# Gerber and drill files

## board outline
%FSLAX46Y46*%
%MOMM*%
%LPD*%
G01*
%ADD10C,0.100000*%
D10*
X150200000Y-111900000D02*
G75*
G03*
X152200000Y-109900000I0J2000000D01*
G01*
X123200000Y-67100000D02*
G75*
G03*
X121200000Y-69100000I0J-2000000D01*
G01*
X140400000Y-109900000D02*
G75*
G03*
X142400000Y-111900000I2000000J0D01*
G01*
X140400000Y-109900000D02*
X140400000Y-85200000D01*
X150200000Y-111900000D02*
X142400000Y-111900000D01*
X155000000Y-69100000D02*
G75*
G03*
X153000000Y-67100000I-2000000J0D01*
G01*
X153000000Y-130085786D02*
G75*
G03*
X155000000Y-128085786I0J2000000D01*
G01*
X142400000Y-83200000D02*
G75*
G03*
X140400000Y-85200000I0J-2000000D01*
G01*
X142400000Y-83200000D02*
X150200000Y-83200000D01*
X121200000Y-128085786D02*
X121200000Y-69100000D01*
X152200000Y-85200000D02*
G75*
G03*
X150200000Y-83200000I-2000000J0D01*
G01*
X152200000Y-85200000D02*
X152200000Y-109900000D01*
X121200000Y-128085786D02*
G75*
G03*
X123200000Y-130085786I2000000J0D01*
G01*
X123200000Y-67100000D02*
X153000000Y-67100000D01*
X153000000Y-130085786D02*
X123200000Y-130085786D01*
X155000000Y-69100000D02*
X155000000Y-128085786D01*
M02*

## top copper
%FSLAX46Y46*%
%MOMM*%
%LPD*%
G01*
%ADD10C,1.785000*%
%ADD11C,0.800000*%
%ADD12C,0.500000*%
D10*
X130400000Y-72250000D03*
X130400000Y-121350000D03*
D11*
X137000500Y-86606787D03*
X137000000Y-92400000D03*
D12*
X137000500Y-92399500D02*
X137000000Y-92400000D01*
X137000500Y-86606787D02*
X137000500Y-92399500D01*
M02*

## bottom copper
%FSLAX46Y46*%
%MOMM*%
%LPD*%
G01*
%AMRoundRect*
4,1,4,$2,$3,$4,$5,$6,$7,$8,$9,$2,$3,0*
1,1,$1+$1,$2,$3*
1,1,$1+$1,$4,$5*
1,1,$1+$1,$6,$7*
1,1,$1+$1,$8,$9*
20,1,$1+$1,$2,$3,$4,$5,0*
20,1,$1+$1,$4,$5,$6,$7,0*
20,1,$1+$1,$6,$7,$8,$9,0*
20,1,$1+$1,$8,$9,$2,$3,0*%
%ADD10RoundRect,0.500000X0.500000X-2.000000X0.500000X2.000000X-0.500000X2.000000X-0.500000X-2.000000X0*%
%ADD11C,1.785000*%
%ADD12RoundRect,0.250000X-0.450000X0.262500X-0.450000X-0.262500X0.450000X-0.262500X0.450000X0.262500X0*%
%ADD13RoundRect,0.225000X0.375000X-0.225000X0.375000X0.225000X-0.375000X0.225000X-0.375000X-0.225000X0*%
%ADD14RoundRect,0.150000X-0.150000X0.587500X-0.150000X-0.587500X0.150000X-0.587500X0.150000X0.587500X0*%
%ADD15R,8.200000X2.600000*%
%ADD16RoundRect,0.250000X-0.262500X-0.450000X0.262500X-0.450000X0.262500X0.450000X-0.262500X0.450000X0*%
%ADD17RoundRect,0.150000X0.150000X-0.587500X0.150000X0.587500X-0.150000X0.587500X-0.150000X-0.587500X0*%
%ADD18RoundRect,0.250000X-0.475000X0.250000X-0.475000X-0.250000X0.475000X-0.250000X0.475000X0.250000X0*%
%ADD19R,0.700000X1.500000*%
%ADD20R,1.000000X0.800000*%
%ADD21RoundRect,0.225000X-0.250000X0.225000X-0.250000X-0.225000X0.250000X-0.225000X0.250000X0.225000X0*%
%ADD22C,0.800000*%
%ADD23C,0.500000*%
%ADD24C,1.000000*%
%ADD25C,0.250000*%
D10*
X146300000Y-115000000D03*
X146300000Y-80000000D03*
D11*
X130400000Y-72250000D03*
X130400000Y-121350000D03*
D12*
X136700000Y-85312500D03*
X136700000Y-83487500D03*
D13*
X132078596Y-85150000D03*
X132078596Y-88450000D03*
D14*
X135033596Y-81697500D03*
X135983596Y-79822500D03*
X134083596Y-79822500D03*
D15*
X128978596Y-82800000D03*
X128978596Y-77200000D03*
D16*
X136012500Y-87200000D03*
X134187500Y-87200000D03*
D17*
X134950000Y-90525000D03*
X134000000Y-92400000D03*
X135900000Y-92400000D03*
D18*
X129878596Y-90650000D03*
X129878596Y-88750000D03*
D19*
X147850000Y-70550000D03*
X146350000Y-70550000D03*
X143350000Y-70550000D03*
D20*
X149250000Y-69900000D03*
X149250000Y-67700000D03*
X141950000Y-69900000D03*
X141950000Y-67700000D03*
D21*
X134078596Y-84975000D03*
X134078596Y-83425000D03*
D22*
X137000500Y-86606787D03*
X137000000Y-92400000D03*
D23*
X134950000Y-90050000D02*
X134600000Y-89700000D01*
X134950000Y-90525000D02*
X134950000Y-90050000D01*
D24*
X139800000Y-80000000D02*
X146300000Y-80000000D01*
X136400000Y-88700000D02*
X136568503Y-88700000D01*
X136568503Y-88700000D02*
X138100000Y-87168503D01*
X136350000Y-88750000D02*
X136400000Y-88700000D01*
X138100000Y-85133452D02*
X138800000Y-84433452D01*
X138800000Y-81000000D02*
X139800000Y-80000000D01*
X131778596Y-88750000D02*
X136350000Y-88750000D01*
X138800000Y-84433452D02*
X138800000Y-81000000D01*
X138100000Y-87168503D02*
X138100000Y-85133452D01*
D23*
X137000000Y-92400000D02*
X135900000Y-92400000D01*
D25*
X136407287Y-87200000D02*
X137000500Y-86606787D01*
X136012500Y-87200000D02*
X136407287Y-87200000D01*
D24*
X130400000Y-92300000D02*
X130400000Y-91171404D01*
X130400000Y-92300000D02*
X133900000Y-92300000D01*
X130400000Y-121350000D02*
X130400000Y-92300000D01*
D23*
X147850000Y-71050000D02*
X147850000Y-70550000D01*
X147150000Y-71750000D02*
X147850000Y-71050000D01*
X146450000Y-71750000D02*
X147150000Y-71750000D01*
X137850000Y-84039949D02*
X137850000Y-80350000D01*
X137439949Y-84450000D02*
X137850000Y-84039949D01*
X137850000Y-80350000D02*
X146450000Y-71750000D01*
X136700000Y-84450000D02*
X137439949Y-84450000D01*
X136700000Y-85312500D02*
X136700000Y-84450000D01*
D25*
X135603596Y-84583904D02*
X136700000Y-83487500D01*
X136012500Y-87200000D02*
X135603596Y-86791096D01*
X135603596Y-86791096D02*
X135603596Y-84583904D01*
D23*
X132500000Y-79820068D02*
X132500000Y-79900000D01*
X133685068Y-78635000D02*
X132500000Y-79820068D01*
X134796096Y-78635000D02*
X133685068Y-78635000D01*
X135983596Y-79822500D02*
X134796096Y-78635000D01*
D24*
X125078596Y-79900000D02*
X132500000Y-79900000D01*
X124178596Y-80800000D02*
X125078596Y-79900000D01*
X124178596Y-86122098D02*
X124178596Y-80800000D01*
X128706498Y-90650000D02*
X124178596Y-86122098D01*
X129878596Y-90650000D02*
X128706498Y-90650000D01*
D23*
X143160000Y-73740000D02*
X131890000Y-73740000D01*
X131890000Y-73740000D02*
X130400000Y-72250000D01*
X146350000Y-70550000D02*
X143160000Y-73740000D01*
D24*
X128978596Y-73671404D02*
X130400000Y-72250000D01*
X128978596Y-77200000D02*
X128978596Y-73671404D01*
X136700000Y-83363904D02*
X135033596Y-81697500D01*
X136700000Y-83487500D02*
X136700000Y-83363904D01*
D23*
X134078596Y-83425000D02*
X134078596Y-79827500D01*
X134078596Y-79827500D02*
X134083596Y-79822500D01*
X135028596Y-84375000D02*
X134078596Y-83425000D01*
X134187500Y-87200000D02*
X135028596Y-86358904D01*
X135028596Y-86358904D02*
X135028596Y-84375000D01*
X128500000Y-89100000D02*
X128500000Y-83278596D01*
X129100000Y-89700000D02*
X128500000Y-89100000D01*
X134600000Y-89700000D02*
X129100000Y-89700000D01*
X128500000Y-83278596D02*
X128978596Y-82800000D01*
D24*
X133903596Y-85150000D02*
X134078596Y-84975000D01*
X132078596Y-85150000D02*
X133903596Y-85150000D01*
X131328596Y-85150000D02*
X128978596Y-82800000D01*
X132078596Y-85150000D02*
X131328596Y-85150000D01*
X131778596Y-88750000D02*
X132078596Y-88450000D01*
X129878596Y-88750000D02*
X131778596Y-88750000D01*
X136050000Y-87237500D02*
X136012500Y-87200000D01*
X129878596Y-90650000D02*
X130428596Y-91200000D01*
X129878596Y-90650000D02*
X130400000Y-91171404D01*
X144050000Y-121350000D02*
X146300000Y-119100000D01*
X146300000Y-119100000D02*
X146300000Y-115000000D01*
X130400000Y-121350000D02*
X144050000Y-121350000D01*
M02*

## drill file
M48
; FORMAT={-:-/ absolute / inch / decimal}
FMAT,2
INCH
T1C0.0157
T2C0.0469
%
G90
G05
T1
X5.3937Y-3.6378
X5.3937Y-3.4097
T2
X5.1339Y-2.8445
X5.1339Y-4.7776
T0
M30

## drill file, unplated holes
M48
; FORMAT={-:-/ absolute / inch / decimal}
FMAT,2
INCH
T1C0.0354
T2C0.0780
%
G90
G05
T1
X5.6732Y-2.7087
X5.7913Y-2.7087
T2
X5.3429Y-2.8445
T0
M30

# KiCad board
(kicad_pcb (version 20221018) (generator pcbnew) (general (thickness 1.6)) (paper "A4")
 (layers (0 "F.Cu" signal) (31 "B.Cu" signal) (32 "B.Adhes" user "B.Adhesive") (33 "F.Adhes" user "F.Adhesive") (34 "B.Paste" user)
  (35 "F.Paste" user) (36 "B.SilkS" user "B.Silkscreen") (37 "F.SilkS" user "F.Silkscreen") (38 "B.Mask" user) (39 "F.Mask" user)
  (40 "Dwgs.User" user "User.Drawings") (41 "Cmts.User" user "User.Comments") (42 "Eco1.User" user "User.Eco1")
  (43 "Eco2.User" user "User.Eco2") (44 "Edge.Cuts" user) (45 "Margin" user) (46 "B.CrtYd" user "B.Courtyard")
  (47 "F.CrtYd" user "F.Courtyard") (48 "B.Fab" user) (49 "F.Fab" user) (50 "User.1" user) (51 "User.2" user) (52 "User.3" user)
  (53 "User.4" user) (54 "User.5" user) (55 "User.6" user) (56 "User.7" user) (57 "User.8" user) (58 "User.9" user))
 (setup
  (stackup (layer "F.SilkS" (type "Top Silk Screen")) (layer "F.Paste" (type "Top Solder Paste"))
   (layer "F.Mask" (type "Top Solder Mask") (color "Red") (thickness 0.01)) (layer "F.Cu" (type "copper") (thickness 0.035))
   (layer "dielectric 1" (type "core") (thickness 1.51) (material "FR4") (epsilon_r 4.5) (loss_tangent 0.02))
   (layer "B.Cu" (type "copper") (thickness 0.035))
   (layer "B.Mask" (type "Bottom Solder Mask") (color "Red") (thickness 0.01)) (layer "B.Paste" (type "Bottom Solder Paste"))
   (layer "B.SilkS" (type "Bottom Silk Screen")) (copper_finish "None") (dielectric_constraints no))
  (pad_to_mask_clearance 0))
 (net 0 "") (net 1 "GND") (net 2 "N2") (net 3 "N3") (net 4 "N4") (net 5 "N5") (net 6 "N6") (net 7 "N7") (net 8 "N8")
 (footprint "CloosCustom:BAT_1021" (layer "F.Cu") (at 130.4 96.8 -90)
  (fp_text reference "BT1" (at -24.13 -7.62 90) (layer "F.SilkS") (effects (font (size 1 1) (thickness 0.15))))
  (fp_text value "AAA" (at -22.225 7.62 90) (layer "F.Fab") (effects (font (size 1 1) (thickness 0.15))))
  (pad "" np_thru_hole circle (at -24.55 -5.31 270) (size 1.98 1.98) (drill 1.98) (layers "*.Cu" "*.Mask"))
  (pad "N" thru_hole circle (at 24.55 0 270) (size 1.785 1.785) (drill 1.19) (layers "*.Cu" "*.Mask") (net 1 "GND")
   (solder_mask_margin 0.102))
  (pad "P" thru_hole circle (at -24.55 0 270) (size 1.785 1.785) (drill 1.19) (layers "*.Cu" "*.Mask") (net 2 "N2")
   (solder_mask_margin 0.102)))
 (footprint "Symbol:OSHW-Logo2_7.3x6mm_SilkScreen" (layer "F.Cu") (at 150.6 78.7)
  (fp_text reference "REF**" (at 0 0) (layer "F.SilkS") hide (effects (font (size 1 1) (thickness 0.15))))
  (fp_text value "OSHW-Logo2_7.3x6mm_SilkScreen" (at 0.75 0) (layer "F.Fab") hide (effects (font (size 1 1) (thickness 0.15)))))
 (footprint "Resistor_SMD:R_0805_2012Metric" (layer "B.Cu") (at 136.7 84.4 -90)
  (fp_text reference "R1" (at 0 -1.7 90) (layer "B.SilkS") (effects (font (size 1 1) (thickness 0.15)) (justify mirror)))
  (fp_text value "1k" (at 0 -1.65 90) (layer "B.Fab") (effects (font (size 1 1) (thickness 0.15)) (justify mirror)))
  (pad "1" smd roundrect (at -0.9125 0 270) (size 1.025 1.4) (layers "B.Cu" "B.Paste" "B.Mask") (roundrect_rratio 0.243902439) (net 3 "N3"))
  (pad "2" smd roundrect (at 0.9125 0 270) (size 1.025 1.4) (layers "B.Cu" "B.Paste" "B.Mask") (roundrect_rratio 0.243902439) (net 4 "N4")))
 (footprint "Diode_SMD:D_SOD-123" (layer "B.Cu") (at 132.078596 86.8 90)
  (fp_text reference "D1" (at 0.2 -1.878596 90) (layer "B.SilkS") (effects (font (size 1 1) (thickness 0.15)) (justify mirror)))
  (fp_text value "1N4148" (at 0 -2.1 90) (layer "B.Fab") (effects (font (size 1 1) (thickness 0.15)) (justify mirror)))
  (pad "1" smd roundrect (at -1.65 0 90) (size 0.9 1.2) (layers "B.Cu" "B.Paste" "B.Mask") (roundrect_rratio 0.25) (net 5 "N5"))
  (pad "2" smd roundrect (at 1.65 0 90) (size 0.9 1.2) (layers "B.Cu" "B.Paste" "B.Mask") (roundrect_rratio 0.25) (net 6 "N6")))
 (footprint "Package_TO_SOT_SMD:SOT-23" (layer "B.Cu") (at 135.033596 80.76 -90)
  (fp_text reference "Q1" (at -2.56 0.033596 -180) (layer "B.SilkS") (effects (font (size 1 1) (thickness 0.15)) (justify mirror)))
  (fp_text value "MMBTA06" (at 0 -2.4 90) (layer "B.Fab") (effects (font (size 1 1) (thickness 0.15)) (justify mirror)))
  (pad "1" smd roundrect (at -0.9375 0.95 270) (size 1.475 0.6) (layers "B.Cu" "B.Paste" "B.Mask") (roundrect_rratio 0.25) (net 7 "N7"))
  (pad "2" smd roundrect (at -0.9375 -0.95 270) (size 1.475 0.6) (layers "B.Cu" "B.Paste" "B.Mask") (roundrect_rratio 0.25) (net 1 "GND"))
  (pad "3" smd roundrect (at 0.9375 0 270) (size 1.475 0.6) (layers "B.Cu" "B.Paste" "B.Mask") (roundrect_rratio 0.25) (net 3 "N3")))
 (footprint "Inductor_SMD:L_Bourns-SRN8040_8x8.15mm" (layer "B.Cu") (at 128.978596 80 90)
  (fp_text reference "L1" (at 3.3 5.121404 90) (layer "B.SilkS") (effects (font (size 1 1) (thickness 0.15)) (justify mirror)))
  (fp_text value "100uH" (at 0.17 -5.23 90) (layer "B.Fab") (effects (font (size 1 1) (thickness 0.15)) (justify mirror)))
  (pad "1" smd rect (at -2.8 0 90) (size 2.6 8.2) (layers "B.Cu" "B.Paste" "B.Mask") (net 6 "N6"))
  (pad "2" smd rect (at 2.8 0 90) (size 2.6 8.2) (layers "B.Cu" "B.Paste" "B.Mask") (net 2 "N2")))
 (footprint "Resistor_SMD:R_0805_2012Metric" (layer "B.Cu") (at 135.1 87.2)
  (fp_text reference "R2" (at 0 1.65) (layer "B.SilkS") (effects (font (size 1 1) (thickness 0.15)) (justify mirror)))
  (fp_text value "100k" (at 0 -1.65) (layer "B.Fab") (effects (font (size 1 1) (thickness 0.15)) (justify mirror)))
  (pad "1" smd roundrect (at -0.9125 0) (size 1.025 1.4) (layers "B.Cu" "B.Paste" "B.Mask") (roundrect_rratio 0.243902439) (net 7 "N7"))
  (pad "2" smd roundrect (at 0.9125 0) (size 1.025 1.4) (layers "B.Cu" "B.Paste" "B.Mask") (roundrect_rratio 0.243902439) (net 3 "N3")))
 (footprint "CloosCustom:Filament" (layer "B.Cu") (at 146.3 117.5 90)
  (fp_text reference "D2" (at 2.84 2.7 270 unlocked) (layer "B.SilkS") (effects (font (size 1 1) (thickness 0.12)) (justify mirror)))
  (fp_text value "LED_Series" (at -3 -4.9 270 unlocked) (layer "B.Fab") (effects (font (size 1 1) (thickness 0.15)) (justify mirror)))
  (pad "1" smd roundrect (at 2.5 0 90) (size 5 2) (layers "B.Cu" "B.Paste" "B.Mask") (roundrect_rratio 0.25) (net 1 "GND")
   (thermal_bridge_angle 45))
  (pad "2" smd roundrect (at 37.5 0 90) (size 5 2) (layers "B.Cu" "B.Paste" "B.Mask") (roundrect_rratio 0.25) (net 5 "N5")
   (thermal_bridge_angle 45)))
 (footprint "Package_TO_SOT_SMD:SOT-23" (layer "B.Cu") (at 134.95 91.4625 90)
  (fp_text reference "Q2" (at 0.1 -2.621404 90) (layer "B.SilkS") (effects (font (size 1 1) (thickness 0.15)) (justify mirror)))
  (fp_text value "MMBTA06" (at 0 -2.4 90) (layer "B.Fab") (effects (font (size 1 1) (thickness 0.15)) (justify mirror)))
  (pad "1" smd roundrect (at -0.9375 0.95 90) (size 1.475 0.6) (layers "B.Cu" "B.Paste" "B.Mask") (roundrect_rratio 0.25) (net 3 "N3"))
  (pad "2" smd roundrect (at -0.9375 -0.95 90) (size 1.475 0.6) (layers "B.Cu" "B.Paste" "B.Mask") (roundrect_rratio 0.25) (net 1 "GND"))
  (pad "3" smd roundrect (at 0.9375 0 90) (size 1.475 0.6) (layers "B.Cu" "B.Paste" "B.Mask") (roundrect_rratio 0.25) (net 6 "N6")))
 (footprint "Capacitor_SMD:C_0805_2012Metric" (layer "B.Cu") (at 129.878596 89.7 -90)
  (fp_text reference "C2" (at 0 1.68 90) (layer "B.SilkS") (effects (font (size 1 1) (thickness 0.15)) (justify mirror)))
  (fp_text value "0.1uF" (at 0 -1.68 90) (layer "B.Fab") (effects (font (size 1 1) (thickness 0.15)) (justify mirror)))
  (pad "1" smd roundrect (at -0.95 0 270) (size 1 1.45) (layers "B.Cu" "B.Paste" "B.Mask") (roundrect_rratio 0.25) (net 5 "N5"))
  (pad "2" smd roundrect (at 0.95 0 270) (size 1 1.45) (layers "B.Cu" "B.Paste" "B.Mask") (roundrect_rratio 0.25) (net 1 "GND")))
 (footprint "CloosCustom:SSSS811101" (layer "B.Cu") (at 145.6 68.8)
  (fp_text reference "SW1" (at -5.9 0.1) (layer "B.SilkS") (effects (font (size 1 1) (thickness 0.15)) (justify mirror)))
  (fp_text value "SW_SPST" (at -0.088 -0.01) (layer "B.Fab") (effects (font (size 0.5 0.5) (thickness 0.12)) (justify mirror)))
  (pad "" smd rect (at -3.65 -1.1) (size 1 0.8) (layers "B.Cu" "B.Paste" "B.Mask"))
  (pad "" smd rect (at -3.65 1.1) (size 1 0.8) (layers "B.Cu" "B.Paste" "B.Mask"))
  (pad "" np_thru_hole circle (at -1.5 0) (size 0.9 0.9) (drill 0.9) (layers "*.Cu" "*.Mask"))
  (pad "" np_thru_hole circle (at 1.5 0) (size 0.9 0.9) (drill 0.9) (layers "*.Cu" "*.Mask"))
  (pad "" smd rect (at 3.65 -1.1) (size 1 0.8) (layers "B.Cu" "B.Paste" "B.Mask"))
  (pad "" smd rect (at 3.65 1.1) (size 1 0.8) (layers "B.Cu" "B.Paste" "B.Mask"))
  (pad "1" smd rect (at -2.25 1.75) (size 0.7 1.5) (layers "B.Cu" "B.Paste" "B.Mask") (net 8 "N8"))
  (pad "2" smd rect (at 0.75 1.75) (size 0.7 1.5) (layers "B.Cu" "B.Paste" "B.Mask") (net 2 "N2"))
  (pad "3" smd rect (at 2.25 1.75) (size 0.7 1.5) (layers "B.Cu" "B.Paste" "B.Mask") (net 4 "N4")))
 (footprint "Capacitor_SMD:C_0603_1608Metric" (layer "B.Cu") (at 134.078596 84.2 -90)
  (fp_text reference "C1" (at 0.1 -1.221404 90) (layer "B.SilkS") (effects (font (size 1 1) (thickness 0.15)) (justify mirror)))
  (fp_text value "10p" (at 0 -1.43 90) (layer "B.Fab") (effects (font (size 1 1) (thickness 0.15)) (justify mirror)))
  (pad "1" smd roundrect (at -0.775 0 270) (size 0.9 0.95) (layers "B.Cu" "B.Paste" "B.Mask") (roundrect_rratio 0.25) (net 7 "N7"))
  (pad "2" smd roundrect (at 0.775 0 270) (size 0.9 0.95) (layers "B.Cu" "B.Paste" "B.Mask") (roundrect_rratio 0.25) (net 6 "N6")))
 (gr_arc (start 152.2 109.9) (mid 151.614214 111.314214) (end 150.2 111.9) (stroke (width 0.1) (type default)) (layer "Edge.Cuts"))
 (gr_arc (start 121.2 69.1) (mid 121.785786 67.685786) (end 123.2 67.1) (stroke (width 0.1) (type default)) (layer "Edge.Cuts"))
 (gr_arc (start 142.4 111.9) (mid 140.985786 111.314214) (end 140.4 109.9) (stroke (width 0.1) (type default)) (layer "Edge.Cuts"))
 (gr_line (start 140.4 109.9) (end 140.4 85.2) (stroke (width 0.1) (type default)) (layer "Edge.Cuts"))
 (gr_line (start 150.2 111.9) (end 142.4 111.9) (stroke (width 0.1) (type default)) (layer "Edge.Cuts"))
 (gr_arc (start 153 67.1) (mid 154.414214 67.685786) (end 155 69.1) (stroke (width 0.1) (type default)) (layer "Edge.Cuts"))
 (gr_arc (start 155 128.085786) (mid 154.414214 129.5) (end 153 130.085786) (stroke (width 0.1) (type default)) (layer "Edge.Cuts"))
 (gr_arc (start 140.4 85.2) (mid 140.985786 83.785786) (end 142.4 83.2) (stroke (width 0.1) (type default)) (layer "Edge.Cuts"))
 (gr_line (start 142.4 83.2) (end 150.2 83.2) (stroke (width 0.1) (type default)) (layer "Edge.Cuts"))
 (gr_line (start 121.2 128.085786) (end 121.2 69.1) (stroke (width 0.1) (type default)) (layer "Edge.Cuts"))
 (gr_arc (start 150.2 83.2) (mid 151.614214 83.785786) (end 152.2 85.2) (stroke (width 0.1) (type default)) (layer "Edge.Cuts"))
 (gr_line (start 152.2 85.2) (end 152.2 109.9) (stroke (width 0.1) (type default)) (layer "Edge.Cuts"))
 (gr_arc (start 123.2 130.085786) (mid 121.785786 129.5) (end 121.2 128.085786) (stroke (width 0.1) (type default)) (layer "Edge.Cuts"))
 (gr_line (start 123.2 67.1) (end 153 67.1) (stroke (width 0.1) (type default)) (layer "Edge.Cuts"))
 (gr_line (start 153 130.085786) (end 123.2 130.085786) (stroke (width 0.1) (type default)) (layer "Edge.Cuts"))
 (gr_line (start 155 69.1) (end 155 128.085786) (stroke (width 0.1) (type default)) (layer "Edge.Cuts"))
 (segment (start 135.028596 84.375) (end 134.078596 83.425) (width 0.5) (layer "B.Cu") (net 7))
 (segment (start 134.078596 79.8275) (end 134.083596 79.8225) (width 0.5) (layer "B.Cu") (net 7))
 (segment (start 135.028596 86.358904) (end 135.028596 84.375) (width 0.5) (layer "B.Cu") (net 7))
 (segment (start 134.078596 83.425) (end 134.078596 79.8275) (width 0.5) (layer "B.Cu") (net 7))
 (segment (start 134.1875 87.2) (end 135.028596 86.358904) (width 0.5) (layer "B.Cu") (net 7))
 (segment (start 134.6 89.7) (end 129.1 89.7) (width 0.5) (layer "B.Cu") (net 6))
 (segment (start 128.5 83.278596) (end 128.978596 82.8) (width 0.5) (layer "B.Cu") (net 6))
 (segment (start 134.95 90.05) (end 134.6 89.7) (width 0.5) (layer "B.Cu") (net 6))
 (segment (start 132.078596 85.15) (end 133.903596 85.15) (width 1) (layer "B.Cu") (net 6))
 (segment (start 132.078596 85.15) (end 131.328596 85.15) (width 1) (layer "B.Cu") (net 6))
 (segment (start 131.328596 85.15) (end 128.978596 82.8) (width 1) (layer "B.Cu") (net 6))
 (segment (start 134.95 90.525) (end 134.95 90.05) (width 0.5) (layer "B.Cu") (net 6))
 (segment (start 129.1 89.7) (end 128.5 89.1) (width 0.5) (layer "B.Cu") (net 6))
 (segment (start 133.903596 85.15) (end 134.078596 84.975) (width 1) (layer "B.Cu") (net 6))
 (segment (start 128.5 89.1) (end 128.5 83.278596) (width 0.5) (layer "B.Cu") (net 6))
 (segment (start 138.8 84.433452) (end 138.8 81) (width 1) (layer "B.Cu") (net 5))
 (segment (start 138.1 87.168503) (end 138.1 85.133452) (width 1) (layer "B.Cu") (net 5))
 (segment (start 136.35 88.75) (end 136.4 88.7) (width 1) (layer "B.Cu") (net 5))
 (segment (start 131.778596 88.75) (end 132.078596 88.45) (width 1) (layer "B.Cu") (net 5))
 (segment (start 136.568503 88.7) (end 138.1 87.168503) (width 1) (layer "B.Cu") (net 5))
 (segment (start 139.8 80) (end 146.3 80) (width 1) (layer "B.Cu") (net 5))
 (segment (start 129.878596 88.75) (end 131.778596 88.75) (width 1) (layer "B.Cu") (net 5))
 (segment (start 138.8 81) (end 139.8 80) (width 1) (layer "B.Cu") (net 5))
 (segment (start 136.4 88.7) (end 136.568503 88.7) (width 1) (layer "B.Cu") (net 5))
 (segment (start 131.778596 88.75) (end 136.35 88.75) (width 1) (layer "B.Cu") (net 5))
 (segment (start 138.1 85.133452) (end 138.8 84.433452) (width 1) (layer "B.Cu") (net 5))
 (segment (start 130.4 92.3) (end 130.4 91.171404) (width 1) (layer "B.Cu") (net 1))
 (segment (start 133.685068 78.635) (end 132.5 79.820068) (width 0.5) (layer "B.Cu") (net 1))
 (segment (start 144.05 121.35) (end 146.3 119.1) (width 1) (layer "B.Cu") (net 1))
 (segment (start 135.983596 79.8225) (end 134.796096 78.635) (width 0.5) (layer "B.Cu") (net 1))
 (segment (start 128.706498 90.65) (end 124.178596 86.122098) (width 1) (layer "B.Cu") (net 1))
 (segment (start 134.796096 78.635) (end 133.685068 78.635) (width 0.5) (layer "B.Cu") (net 1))
 (segment (start 125.078596 79.9) (end 132.5 79.9) (width 1) (layer "B.Cu") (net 1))
 (segment (start 130.4 92.3) (end 133.9 92.3) (width 1) (layer "B.Cu") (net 1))
 (segment (start 124.178596 80.8) (end 125.078596 79.9) (width 1) (layer "B.Cu") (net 1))
 (segment (start 130.4 121.35) (end 130.4 92.3) (width 1) (layer "B.Cu") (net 1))
 (segment (start 132.5 79.820068) (end 132.5 79.9) (width 0.5) (layer "B.Cu") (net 1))
 (segment (start 124.178596 86.122098) (end 124.178596 80.8) (width 1) (layer "B.Cu") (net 1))
 (segment (start 129.878596 90.65) (end 130.428596 91.2) (width 1) (layer "B.Cu") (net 1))
 (segment (start 130.4 121.35) (end 144.05 121.35) (width 1) (layer "B.Cu") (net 1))
 (segment (start 129.878596 90.65) (end 130.4 91.171404) (width 1) (layer "B.Cu") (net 1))
 (segment (start 129.878596 90.65) (end 128.706498 90.65) (width 1) (layer "B.Cu") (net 1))
 (segment (start 146.3 119.1) (end 146.3 115) (width 1) (layer "B.Cu") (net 1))
 (segment (start 137.0005 92.3995) (end 137 92.4) (width 0.5) (layer "F.Cu") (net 3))
 (segment (start 137.0005 86.606787) (end 137.0005 92.3995) (width 0.5) (layer "F.Cu") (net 3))
 (via (at 137 92.4) (size 0.8) (drill 0.4) (layers "F.Cu" "B.Cu") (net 3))
 (via (at 137.0005 86.606787) (size 0.8) (drill 0.4) (layers "F.Cu" "B.Cu") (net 3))
 (segment (start 136.0125 87.2) (end 135.603596 86.791096) (width 0.25) (layer "B.Cu") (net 3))
 (segment (start 136.7 83.4875) (end 136.7 83.363904) (width 1) (layer "B.Cu") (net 3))
 (segment (start 136.7 83.363904) (end 135.033596 81.6975) (width 1) (layer "B.Cu") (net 3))
 (segment (start 135.603596 84.583904) (end 136.7 83.4875) (width 0.25) (layer "B.Cu") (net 3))
 (segment (start 136.407287 87.2) (end 137.0005 86.606787) (width 0.25) (layer "B.Cu") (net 3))
 (segment (start 136.05 87.2375) (end 136.0125 87.2) (width 1) (layer "B.Cu") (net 3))
 (segment (start 136.0125 87.2) (end 136.407287 87.2) (width 0.25) (layer "B.Cu") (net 3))
 (segment (start 135.603596 86.791096) (end 135.603596 84.583904) (width 0.25) (layer "B.Cu") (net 3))
 (segment (start 137 92.4) (end 135.9 92.4) (width 0.5) (layer "B.Cu") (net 3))
 (segment (start 146.35 70.55) (end 143.16 73.74) (width 0.5) (layer "B.Cu") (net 2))
 (segment (start 131.89 73.74) (end 130.4 72.25) (width 0.5) (layer "B.Cu") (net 2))
 (segment (start 128.978596 73.671404) (end 130.4 72.25) (width 1) (layer "B.Cu") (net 2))
 (segment (start 143.16 73.74) (end 131.89 73.74) (width 0.5) (layer "B.Cu") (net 2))
 (segment (start 128.978596 77.2) (end 128.978596 73.671404) (width 1) (layer "B.Cu") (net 2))
 (segment (start 137.85 80.35) (end 146.45 71.75) (width 0.5) (layer "B.Cu") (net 4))
 (segment (start 137.439949 84.45) (end 137.85 84.039949) (width 0.5) (layer "B.Cu") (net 4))
 (segment (start 136.7 85.3125) (end 136.7 84.45) (width 0.5) (layer "B.Cu") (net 4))
 (segment (start 146.45 71.75) (end 147.15 71.75) (width 0.5) (layer "B.Cu") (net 4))
 (segment (start 147.85 71.05) (end 147.85 70.55) (width 0.5) (layer "B.Cu") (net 4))
 (segment (start 137.85 84.039949) (end 137.85 80.35) (width 0.5) (layer "B.Cu") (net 4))
 (segment (start 147.15 71.75) (end 147.85 71.05) (width 0.5) (layer "B.Cu") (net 4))
 (segment (start 136.7 84.45) (end 137.439949 84.45) (width 0.5) (layer "B.Cu") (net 4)))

